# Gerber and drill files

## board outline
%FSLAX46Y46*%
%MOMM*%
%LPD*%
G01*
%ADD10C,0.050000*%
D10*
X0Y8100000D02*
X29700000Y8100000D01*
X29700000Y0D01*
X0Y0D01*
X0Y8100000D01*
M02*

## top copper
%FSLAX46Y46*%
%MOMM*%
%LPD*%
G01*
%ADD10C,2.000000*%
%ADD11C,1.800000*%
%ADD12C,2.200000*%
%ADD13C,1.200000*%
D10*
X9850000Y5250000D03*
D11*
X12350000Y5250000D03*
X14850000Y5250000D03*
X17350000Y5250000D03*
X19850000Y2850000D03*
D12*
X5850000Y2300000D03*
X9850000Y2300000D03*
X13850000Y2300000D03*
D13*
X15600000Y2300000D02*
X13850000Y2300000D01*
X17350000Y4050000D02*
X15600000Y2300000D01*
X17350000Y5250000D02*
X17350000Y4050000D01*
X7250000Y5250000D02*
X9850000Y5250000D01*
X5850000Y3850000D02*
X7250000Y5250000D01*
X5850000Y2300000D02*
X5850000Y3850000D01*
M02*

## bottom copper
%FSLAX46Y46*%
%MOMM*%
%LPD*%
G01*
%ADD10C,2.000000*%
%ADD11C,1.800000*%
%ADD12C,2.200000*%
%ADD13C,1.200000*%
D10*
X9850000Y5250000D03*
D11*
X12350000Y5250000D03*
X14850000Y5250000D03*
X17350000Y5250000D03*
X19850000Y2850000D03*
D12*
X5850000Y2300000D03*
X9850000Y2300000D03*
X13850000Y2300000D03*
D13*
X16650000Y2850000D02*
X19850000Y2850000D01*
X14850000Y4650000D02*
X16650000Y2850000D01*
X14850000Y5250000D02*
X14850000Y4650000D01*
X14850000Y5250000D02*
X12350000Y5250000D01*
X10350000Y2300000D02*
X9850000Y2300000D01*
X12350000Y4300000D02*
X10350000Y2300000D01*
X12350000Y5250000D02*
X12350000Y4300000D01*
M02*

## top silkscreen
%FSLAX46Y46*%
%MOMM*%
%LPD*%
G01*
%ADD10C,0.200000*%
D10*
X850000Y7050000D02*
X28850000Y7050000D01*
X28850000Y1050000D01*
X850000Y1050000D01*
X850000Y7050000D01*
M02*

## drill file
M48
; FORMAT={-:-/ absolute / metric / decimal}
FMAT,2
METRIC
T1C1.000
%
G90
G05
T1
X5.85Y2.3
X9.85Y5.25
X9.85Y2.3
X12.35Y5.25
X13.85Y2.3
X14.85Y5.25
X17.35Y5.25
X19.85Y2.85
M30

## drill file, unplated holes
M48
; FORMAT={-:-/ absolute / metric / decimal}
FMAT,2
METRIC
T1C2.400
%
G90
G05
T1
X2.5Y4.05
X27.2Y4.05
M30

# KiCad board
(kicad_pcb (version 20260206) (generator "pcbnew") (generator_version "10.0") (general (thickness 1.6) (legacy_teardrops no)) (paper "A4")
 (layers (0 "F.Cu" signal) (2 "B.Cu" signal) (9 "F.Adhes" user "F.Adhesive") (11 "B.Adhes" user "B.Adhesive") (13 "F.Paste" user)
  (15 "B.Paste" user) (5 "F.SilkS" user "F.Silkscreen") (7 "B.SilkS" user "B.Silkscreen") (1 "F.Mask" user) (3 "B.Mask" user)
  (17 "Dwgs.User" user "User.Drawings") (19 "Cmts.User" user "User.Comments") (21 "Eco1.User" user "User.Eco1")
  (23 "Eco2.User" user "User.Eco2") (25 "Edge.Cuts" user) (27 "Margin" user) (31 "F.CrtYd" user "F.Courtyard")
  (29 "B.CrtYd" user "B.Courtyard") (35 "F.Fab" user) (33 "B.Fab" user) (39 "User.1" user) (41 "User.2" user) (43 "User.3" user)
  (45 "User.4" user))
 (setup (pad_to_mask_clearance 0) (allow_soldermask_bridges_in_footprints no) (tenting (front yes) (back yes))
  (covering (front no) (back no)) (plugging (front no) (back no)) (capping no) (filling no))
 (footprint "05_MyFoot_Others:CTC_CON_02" (layer "F.Cu") (at 14.85 -4.05)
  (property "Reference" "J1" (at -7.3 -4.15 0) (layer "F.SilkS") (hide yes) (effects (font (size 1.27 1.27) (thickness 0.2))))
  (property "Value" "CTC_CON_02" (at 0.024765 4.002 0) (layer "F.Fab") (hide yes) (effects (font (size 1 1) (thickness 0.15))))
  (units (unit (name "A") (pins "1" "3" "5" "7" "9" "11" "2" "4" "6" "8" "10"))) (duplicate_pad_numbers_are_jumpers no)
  (fp_rect (start -14 -3) (end 14 3) (stroke (width 0.2) (type default)) (fill no) (layer "F.SilkS"))
  (pad "" np_thru_hole circle (at -12.35 0) (size 2.4 2.4) (drill 2.4) (layers "*.Cu") (thermal_bridge_angle 90))
  (pad "" np_thru_hole circle (at 12.35 0) (size 2.4 2.4) (drill 2.4) (layers "*.Cu") (thermal_bridge_angle 90))
  (pad "1" thru_hole circle (at -5 -1.2) (size 2 2) (drill 1) (layers "*.Cu" "*.Mask") (remove_unused_layers no) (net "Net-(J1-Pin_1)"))
  (pad "2" thru_hole circle (at -2.5 -1.2) (size 1.8 1.8) (drill 1) (layers "*.Cu" "*.Mask") (remove_unused_layers no)
   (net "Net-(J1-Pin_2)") (thermal_bridge_angle 90))
  (pad "3" thru_hole circle (at 0 -1.2) (size 1.8 1.8) (drill 1) (layers "*.Cu" "*.Mask") (remove_unused_layers no) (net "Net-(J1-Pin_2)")
   (thermal_bridge_angle 90))
  (pad "4" thru_hole circle (at 2.5 -1.2) (size 1.8 1.8) (drill 1) (layers "*.Cu" "*.Mask") (remove_unused_layers no) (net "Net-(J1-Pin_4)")
   (thermal_bridge_angle 90))
  (pad "5" thru_hole circle (at 5 1.2) (size 1.8 1.8) (drill 1) (layers "*.Cu" "*.Mask") (remove_unused_layers no) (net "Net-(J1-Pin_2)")
   (thermal_bridge_angle 90))
  (pad "6" thru_hole circle (at -9 1.75) (size 2.2 2.2) (drill 1) (layers "*.Cu" "*.Mask") (remove_unused_layers no) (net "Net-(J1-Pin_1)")
   (thermal_bridge_angle 90))
  (pad "7" thru_hole circle (at -5 1.75) (size 2.2 2.2) (drill 1) (layers "*.Cu" "*.Mask") (remove_unused_layers no) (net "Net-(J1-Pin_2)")
   (thermal_bridge_angle 90))
  (pad "8" thru_hole circle (at -1 1.75) (size 2.2 2.2) (drill 1) (layers "*.Cu" "*.Mask") (remove_unused_layers no) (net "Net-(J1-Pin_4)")
   (thermal_bridge_angle 90)))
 (gr_rect (start 0 0) (end 29.7 -8.1) (stroke (width 0.05) (type solid)) (fill no) (layer "Edge.Cuts"))
 (segment (start 7.25 -5.25) (end 9.85 -5.25) (width 1.2) (layer "F.Cu") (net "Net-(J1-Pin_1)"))
 (segment (start 5.85 -2.3) (end 5.85 -3.85) (width 1.2) (layer "F.Cu") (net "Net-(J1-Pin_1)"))
 (segment (start 5.85 -3.85) (end 7.25 -5.25) (width 1.2) (layer "F.Cu") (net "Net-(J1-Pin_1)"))
 (segment (start 17.35 -4.05) (end 15.6 -2.3) (width 1.2) (layer "F.Cu") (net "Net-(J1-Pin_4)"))
 (segment (start 15.6 -2.3) (end 13.85 -2.3) (width 1.2) (layer "F.Cu") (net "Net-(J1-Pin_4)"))
 (segment (start 17.35 -5.25) (end 17.35 -4.05) (width 1.2) (layer "F.Cu") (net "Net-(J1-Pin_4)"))
 (segment (start 12.35 -5.25) (end 12.35 -4.3) (width 1.2) (layer "B.Cu") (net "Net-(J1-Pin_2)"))
 (segment (start 16.65 -2.85) (end 19.85 -2.85) (width 1.2) (layer "B.Cu") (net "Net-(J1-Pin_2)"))
 (segment (start 14.85 -4.65) (end 16.65 -2.85) (width 1.2) (layer "B.Cu") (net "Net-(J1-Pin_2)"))
 (segment (start 14.85 -5.25) (end 12.35 -5.25) (width 1.2) (layer "B.Cu") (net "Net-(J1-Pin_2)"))
 (segment (start 12.35 -4.3) (end 10.35 -2.3) (width 1.2) (layer "B.Cu") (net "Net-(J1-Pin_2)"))
 (segment (start 14.85 -5.25) (end 14.85 -4.65) (width 1.2) (layer "B.Cu") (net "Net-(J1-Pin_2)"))
 (segment (start 10.35 -2.3) (end 9.85 -2.3) (width 1.2) (layer "B.Cu") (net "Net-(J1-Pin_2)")))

